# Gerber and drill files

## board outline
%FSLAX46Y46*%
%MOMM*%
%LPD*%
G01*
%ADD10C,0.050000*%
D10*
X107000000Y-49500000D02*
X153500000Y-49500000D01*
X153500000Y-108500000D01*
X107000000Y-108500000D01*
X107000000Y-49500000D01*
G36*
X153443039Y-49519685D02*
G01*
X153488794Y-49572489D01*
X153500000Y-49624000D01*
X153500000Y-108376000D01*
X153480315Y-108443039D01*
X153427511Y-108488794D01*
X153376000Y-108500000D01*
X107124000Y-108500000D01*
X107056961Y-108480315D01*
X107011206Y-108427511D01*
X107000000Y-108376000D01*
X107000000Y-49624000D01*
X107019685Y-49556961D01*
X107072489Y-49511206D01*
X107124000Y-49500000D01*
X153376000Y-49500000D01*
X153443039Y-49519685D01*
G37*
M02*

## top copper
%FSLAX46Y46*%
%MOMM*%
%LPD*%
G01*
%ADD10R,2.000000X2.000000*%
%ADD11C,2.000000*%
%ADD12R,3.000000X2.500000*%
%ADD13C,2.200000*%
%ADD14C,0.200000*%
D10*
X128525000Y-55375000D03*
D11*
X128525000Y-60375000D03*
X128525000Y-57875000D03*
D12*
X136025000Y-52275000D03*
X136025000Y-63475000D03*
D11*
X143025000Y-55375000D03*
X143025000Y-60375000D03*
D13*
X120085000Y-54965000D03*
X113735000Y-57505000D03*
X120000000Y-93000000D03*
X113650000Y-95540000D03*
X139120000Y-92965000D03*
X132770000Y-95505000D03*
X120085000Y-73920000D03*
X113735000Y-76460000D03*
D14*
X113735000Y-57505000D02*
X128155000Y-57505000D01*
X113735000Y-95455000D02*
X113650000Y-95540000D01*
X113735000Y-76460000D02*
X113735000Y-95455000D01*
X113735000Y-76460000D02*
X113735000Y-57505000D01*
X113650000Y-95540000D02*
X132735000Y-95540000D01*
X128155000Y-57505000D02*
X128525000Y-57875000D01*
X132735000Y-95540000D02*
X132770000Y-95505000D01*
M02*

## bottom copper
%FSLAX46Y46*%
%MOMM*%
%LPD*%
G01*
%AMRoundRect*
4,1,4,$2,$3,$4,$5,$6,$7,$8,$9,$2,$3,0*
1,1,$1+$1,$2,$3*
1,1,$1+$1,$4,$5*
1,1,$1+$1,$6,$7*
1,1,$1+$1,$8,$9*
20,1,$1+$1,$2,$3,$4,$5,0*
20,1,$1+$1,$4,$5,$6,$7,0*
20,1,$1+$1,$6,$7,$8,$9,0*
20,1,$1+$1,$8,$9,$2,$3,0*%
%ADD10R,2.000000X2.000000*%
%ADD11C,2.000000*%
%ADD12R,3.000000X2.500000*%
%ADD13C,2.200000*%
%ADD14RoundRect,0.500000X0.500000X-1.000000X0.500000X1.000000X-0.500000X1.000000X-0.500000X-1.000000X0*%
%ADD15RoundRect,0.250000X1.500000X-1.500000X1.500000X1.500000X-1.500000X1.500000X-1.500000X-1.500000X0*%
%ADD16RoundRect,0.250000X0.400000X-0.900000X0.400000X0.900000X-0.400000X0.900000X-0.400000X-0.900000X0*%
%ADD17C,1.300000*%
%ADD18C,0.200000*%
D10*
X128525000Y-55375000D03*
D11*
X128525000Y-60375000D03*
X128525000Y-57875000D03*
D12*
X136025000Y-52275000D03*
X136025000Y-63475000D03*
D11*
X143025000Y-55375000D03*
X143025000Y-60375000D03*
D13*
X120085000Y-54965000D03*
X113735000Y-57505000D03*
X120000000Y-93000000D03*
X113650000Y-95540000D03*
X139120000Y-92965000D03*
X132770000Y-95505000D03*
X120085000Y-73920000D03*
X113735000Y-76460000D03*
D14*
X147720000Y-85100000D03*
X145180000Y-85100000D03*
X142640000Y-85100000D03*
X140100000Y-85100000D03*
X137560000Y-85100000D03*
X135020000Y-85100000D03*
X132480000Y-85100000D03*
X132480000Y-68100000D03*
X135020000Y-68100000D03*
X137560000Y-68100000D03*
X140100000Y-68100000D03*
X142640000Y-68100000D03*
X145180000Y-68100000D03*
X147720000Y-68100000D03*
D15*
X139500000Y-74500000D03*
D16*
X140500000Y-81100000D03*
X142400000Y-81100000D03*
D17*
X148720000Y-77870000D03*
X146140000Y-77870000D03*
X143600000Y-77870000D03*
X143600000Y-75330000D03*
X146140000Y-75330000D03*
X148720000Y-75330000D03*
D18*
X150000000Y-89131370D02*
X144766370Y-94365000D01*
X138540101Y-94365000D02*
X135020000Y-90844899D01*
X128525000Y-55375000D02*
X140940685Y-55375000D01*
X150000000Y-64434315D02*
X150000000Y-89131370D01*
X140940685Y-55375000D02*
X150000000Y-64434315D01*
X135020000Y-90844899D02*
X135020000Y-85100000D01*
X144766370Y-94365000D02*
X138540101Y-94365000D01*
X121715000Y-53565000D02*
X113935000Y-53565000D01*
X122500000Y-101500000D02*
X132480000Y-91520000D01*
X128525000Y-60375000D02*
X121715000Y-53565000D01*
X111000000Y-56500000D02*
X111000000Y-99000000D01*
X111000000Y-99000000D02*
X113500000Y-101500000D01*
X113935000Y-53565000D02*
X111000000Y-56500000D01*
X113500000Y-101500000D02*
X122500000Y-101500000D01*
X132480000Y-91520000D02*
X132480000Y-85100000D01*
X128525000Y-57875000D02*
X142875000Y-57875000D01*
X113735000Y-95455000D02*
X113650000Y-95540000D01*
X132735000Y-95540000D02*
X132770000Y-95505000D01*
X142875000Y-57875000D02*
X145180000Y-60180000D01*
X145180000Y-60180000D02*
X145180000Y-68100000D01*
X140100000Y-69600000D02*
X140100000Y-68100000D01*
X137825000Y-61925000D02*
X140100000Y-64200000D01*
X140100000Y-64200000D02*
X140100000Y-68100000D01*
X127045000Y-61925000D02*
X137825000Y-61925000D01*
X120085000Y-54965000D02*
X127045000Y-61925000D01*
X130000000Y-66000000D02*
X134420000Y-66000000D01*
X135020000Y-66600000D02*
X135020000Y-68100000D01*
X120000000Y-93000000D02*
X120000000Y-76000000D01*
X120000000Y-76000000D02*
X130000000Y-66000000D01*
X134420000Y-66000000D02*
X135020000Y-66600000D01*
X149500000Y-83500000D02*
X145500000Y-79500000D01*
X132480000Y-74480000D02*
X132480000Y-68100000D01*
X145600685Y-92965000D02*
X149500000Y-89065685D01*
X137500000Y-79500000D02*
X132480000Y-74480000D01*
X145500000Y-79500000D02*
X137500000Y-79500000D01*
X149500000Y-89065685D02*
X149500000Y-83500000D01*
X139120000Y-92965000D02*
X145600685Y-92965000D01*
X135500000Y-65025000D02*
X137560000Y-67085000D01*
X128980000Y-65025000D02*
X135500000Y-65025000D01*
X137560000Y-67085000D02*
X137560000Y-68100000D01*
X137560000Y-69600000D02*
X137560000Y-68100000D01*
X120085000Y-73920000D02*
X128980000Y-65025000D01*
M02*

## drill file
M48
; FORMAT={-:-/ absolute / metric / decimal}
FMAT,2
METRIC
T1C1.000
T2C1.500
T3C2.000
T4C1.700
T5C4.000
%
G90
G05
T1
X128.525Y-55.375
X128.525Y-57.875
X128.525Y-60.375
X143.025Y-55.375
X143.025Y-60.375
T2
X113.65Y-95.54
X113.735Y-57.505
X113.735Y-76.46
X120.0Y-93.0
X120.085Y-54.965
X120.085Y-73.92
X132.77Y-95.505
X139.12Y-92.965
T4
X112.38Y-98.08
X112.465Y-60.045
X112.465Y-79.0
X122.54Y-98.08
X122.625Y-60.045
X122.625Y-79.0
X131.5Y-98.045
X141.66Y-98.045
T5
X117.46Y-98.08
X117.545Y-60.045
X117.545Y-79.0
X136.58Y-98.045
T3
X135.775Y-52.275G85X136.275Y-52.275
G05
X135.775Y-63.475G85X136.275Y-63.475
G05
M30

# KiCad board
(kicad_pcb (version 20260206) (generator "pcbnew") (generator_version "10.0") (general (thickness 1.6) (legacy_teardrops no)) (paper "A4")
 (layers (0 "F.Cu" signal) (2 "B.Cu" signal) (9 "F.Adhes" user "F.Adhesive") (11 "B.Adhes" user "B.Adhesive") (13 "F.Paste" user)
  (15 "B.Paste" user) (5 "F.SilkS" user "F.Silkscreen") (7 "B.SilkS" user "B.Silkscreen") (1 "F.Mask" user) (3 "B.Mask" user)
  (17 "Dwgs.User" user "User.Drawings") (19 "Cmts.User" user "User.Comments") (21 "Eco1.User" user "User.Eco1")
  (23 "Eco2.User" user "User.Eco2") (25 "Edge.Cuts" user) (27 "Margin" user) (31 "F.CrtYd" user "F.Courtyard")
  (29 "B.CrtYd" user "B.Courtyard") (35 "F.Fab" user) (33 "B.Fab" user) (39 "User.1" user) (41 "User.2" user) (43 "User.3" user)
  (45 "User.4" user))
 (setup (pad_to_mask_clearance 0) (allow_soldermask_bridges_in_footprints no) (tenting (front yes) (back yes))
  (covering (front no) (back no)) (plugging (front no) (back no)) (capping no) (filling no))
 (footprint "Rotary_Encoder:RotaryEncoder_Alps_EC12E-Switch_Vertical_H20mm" (layer "F.Cu") (at 128.525 55.375)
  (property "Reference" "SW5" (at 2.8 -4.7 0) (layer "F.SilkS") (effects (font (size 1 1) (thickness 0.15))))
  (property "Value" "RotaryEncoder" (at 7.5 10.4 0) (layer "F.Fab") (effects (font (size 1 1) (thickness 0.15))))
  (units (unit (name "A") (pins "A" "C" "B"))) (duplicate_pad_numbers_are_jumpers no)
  (pad "A" thru_hole rect (at 0 0) (size 2 2) (drill 1) (layers "*.Cu" "*.Mask") (remove_unused_layers no) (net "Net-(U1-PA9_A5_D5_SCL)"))
  (pad "B" thru_hole circle (at 0 5) (size 2 2) (drill 1) (layers "*.Cu" "*.Mask") (remove_unused_layers no) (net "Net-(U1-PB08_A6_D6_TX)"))
  (pad "C" thru_hole circle (at 0 2.5) (size 2 2) (drill 1) (layers "*.Cu" "*.Mask") (remove_unused_layers no) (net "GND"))
  (pad "MP" thru_hole rect (at 7.5 -3.1) (size 3 2.5) (drill oval 2.5 2) (layers "*.Cu" "*.Mask") (remove_unused_layers no))
  (pad "MP" thru_hole rect (at 7.5 8.1) (size 3 2.5) (drill oval 2.5 2) (layers "*.Cu" "*.Mask") (remove_unused_layers no))
  (pad "S1" thru_hole circle (at 14.5 0) (size 2 2) (drill 1) (layers "*.Cu" "*.Mask") (remove_unused_layers no))
  (pad "S2" thru_hole circle (at 14.5 5) (size 2 2) (drill 1) (layers "*.Cu" "*.Mask") (remove_unused_layers no)))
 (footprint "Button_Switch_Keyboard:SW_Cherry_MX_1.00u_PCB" (layer "F.Cu") (at 120.085 54.965)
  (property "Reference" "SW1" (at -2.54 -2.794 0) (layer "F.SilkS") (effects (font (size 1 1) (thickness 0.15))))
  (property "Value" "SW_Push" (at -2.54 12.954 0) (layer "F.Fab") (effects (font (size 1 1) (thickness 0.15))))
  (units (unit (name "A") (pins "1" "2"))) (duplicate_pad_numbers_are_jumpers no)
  (pad "" np_thru_hole circle (at -7.62 5.08) (size 1.7 1.7) (drill 1.7) (layers "*.Cu" "*.Mask"))
  (pad "" np_thru_hole circle (at -2.54 5.08) (size 4 4) (drill 4) (layers "*.Cu" "*.Mask"))
  (pad "" np_thru_hole circle (at 2.54 5.08) (size 1.7 1.7) (drill 1.7) (layers "*.Cu" "*.Mask"))
  (pad "1" thru_hole circle (at 0 0) (size 2.2 2.2) (drill 1.5) (layers "*.Cu" "*.Mask") (remove_unused_layers no)
   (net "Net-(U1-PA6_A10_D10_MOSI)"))
  (pad "2" thru_hole circle (at -6.35 2.54) (size 2.2 2.2) (drill 1.5) (layers "*.Cu" "*.Mask") (remove_unused_layers no) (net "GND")))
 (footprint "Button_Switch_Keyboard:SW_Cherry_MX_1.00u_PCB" (layer "F.Cu") (at 120 93)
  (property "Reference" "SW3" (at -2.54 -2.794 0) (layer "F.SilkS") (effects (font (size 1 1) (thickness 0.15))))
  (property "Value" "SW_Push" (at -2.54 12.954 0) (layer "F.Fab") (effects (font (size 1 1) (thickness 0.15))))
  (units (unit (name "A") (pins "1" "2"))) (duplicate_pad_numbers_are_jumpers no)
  (pad "" np_thru_hole circle (at -7.62 5.08) (size 1.7 1.7) (drill 1.7) (layers "*.Cu" "*.Mask"))
  (pad "" np_thru_hole circle (at -2.54 5.08) (size 4 4) (drill 4) (layers "*.Cu" "*.Mask"))
  (pad "" np_thru_hole circle (at 2.54 5.08) (size 1.7 1.7) (drill 1.7) (layers "*.Cu" "*.Mask"))
  (pad "1" thru_hole circle (at 0 0) (size 2.2 2.2) (drill 1.5) (layers "*.Cu" "*.Mask") (remove_unused_layers no)
   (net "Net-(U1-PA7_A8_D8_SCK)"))
  (pad "2" thru_hole circle (at -6.35 2.54) (size 2.2 2.2) (drill 1.5) (layers "*.Cu" "*.Mask") (remove_unused_layers no) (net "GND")))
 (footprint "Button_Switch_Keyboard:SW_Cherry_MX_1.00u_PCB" (layer "F.Cu") (at 139.12 92.965)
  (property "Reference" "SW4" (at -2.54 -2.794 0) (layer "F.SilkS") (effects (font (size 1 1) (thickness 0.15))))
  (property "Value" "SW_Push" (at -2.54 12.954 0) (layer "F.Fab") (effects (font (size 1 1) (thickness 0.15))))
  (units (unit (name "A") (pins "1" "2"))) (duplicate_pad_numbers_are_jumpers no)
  (pad "" np_thru_hole circle (at -7.62 5.08) (size 1.7 1.7) (drill 1.7) (layers "*.Cu" "*.Mask"))
  (pad "" np_thru_hole circle (at -2.54 5.08) (size 4 4) (drill 4) (layers "*.Cu" "*.Mask"))
  (pad "" np_thru_hole circle (at 2.54 5.08) (size 1.7 1.7) (drill 1.7) (layers "*.Cu" "*.Mask"))
  (pad "1" thru_hole circle (at 0 0) (size 2.2 2.2) (drill 1.5) (layers "*.Cu" "*.Mask") (remove_unused_layers no)
   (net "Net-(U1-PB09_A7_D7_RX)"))
  (pad "2" thru_hole circle (at -6.35 2.54) (size 2.2 2.2) (drill 1.5) (layers "*.Cu" "*.Mask") (remove_unused_layers no) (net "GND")))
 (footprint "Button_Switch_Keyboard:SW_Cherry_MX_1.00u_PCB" (layer "F.Cu") (at 120.085 73.92)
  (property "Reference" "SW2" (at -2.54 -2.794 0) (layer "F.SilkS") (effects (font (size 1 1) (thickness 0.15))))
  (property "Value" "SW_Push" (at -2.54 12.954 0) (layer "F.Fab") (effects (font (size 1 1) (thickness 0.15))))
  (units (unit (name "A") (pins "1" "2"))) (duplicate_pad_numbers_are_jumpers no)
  (pad "" np_thru_hole circle (at -7.62 5.08) (size 1.7 1.7) (drill 1.7) (layers "*.Cu" "*.Mask"))
  (pad "" np_thru_hole circle (at -2.54 5.08) (size 4 4) (drill 4) (layers "*.Cu" "*.Mask"))
  (pad "" np_thru_hole circle (at 2.54 5.08) (size 1.7 1.7) (drill 1.7) (layers "*.Cu" "*.Mask"))
  (pad "1" thru_hole circle (at 0 0) (size 2.2 2.2) (drill 1.5) (layers "*.Cu" "*.Mask") (remove_unused_layers no)
   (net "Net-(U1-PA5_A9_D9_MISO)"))
  (pad "2" thru_hole circle (at -6.35 2.54) (size 2.2 2.2) (drill 1.5) (layers "*.Cu" "*.Mask") (remove_unused_layers no) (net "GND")))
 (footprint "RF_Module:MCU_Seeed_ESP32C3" (layer "B.Cu") (at 140.1 76.6 90)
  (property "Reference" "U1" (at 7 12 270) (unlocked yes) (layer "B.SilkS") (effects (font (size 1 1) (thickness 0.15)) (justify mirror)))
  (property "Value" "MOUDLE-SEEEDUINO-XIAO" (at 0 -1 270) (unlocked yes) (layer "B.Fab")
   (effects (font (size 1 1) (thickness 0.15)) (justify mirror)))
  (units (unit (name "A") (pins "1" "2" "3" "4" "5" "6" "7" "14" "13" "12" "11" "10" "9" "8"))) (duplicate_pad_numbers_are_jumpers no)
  (pad "" smd roundrect (at 1.1 -1.6 90) (size 1.5 1.5) (layers "B.Paste") (roundrect_rratio 0.1666666667))
  (pad "" smd roundrect (at 1.1 0.4 90) (size 1.5 1.5) (layers "B.Paste") (roundrect_rratio 0.1666666667))
  (pad "" smd roundrect (at 3.1 -1.6 90) (size 1.5 1.5) (layers "B.Paste") (roundrect_rratio 0.1666666667))
  (pad "" smd roundrect (at 3.1 0.4 90) (size 1.5 1.5) (layers "B.Paste") (roundrect_rratio 0.1666666667))
  (pad "1" smd roundrect (at -8.5 7.62 90) (size 3 2) (layers "B.Cu" "B.Mask" "B.Paste") (roundrect_rratio 0.25)
   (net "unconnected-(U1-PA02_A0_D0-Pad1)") (thermal_bridge_angle 45))
  (pad "2" smd roundrect (at -8.5 5.08 90) (size 3 2) (layers "B.Cu" "B.Mask" "B.Paste") (roundrect_rratio 0.25)
   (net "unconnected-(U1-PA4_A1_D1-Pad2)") (thermal_bridge_angle 45))
  (pad "3" smd roundrect (at -8.5 2.54 90) (size 3 2) (layers "B.Cu" "B.Mask" "B.Paste") (roundrect_rratio 0.25)
   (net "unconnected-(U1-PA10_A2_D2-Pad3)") (thermal_bridge_angle 45))
  (pad "4" smd roundrect (at -8.5 0 90) (size 3 2) (layers "B.Cu" "B.Mask" "B.Paste") (roundrect_rratio 0.25)
   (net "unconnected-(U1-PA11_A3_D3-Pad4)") (thermal_bridge_angle 45))
  (pad "5" smd roundrect (at -8.5 -2.54 90) (size 3 2) (layers "B.Cu" "B.Mask" "B.Paste") (roundrect_rratio 0.25)
   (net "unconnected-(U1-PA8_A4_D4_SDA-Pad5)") (thermal_bridge_angle 45))
  (pad "6" smd roundrect (at -8.5 -5.08 90) (size 3 2) (layers "B.Cu" "B.Mask" "B.Paste") (roundrect_rratio 0.25)
   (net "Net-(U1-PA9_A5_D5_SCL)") (thermal_bridge_angle 45))
  (pad "7" smd roundrect (at -8.5 -7.62 90) (size 3 2) (layers "B.Cu" "B.Mask" "B.Paste") (roundrect_rratio 0.25)
   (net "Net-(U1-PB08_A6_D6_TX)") (thermal_bridge_angle 45))
  (pad "8" smd roundrect (at 8.5 -7.62 90) (size 3 2) (layers "B.Cu" "B.Mask" "B.Paste") (roundrect_rratio 0.25)
   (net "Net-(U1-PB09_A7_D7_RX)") (thermal_bridge_angle 45))
  (pad "9" smd roundrect (at 8.5 -5.08 90) (size 3 2) (layers "B.Cu" "B.Mask" "B.Paste") (roundrect_rratio 0.25)
   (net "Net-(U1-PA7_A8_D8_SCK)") (thermal_bridge_angle 45))
  (pad "10" smd roundrect (at 8.5 -2.54 90) (size 3 2) (layers "B.Cu" "B.Mask" "B.Paste") (roundrect_rratio 0.25)
   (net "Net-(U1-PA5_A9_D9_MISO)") (thermal_bridge_angle 45))
  (pad "11" smd roundrect (at 8.5 0 90) (size 3 2) (layers "B.Cu" "B.Mask" "B.Paste") (roundrect_rratio 0.25)
   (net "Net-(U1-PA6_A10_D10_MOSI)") (thermal_bridge_angle 45))
  (pad "12" smd roundrect (at 8.5 2.54 90) (size 3 2) (layers "B.Cu" "B.Mask" "B.Paste") (roundrect_rratio 0.25)
   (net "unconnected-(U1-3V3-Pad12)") (thermal_bridge_angle 45))
  (pad "13" smd roundrect (at 8.5 5.08 90) (size 3 2) (layers "B.Cu" "B.Mask" "B.Paste") (roundrect_rratio 0.25) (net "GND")
   (thermal_bridge_angle 45))
  (pad "14" smd roundrect (at 8.5 7.62 90) (size 3 2) (layers "B.Cu" "B.Mask" "B.Paste") (roundrect_rratio 0.25)
   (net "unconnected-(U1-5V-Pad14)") (thermal_bridge_angle 45))
  (pad "15" smd roundrect (at 2.1 -0.6 90) (size 3.5 3.5) (layers "B.Cu" "B.Mask") (roundrect_rratio 0.07142857143))
  (pad "16" smd roundrect (at -4.5 0.4 90) (size 2.3 1.3) (layers "B.Cu" "B.Mask" "B.Paste") (roundrect_rratio 0.1923076923))
  (pad "17" smd roundrect (at -4.5 2.3 90) (size 2.3 1.3) (layers "B.Cu" "B.Mask" "B.Paste") (roundrect_rratio 0.1923076923))
  (pad "18" smd circle (at -1.27 8.62 90) (size 1.3 1.3) (layers "B.Cu" "B.Mask" "B.Paste"))
  (pad "19" smd circle (at -1.27 6.04 90) (size 1.3 1.3) (layers "B.Cu" "B.Mask" "B.Paste"))
  (pad "20" smd circle (at -1.27 3.5 90) (size 1.3 1.3) (layers "B.Cu" "B.Mask" "B.Paste"))
  (pad "21" smd circle (at 1.27 3.5 90) (size 1.3 1.3) (layers "B.Cu" "B.Mask" "B.Paste"))
  (pad "22" smd circle (at 1.27 6.04 90) (size 1.3 1.3) (layers "B.Cu" "B.Mask" "B.Paste"))
  (pad "23" smd circle (at 1.27 8.62 90) (size 1.3 1.3) (layers "B.Cu" "B.Mask" "B.Paste")))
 (gr_rect (start 107 49.5) (end 153.5 108.5) (stroke (width 0.05) (type default)) (fill no) (layer "Edge.Cuts"))
 (segment (start 150 89.13137) (end 144.76637 94.365) (width 0.2) (layer "B.Cu") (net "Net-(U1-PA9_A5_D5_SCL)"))
 (segment (start 138.540101 94.365) (end 135.02 90.844899) (width 0.2) (layer "B.Cu") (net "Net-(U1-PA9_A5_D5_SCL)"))
 (segment (start 128.525 55.375) (end 140.940685 55.375) (width 0.2) (layer "B.Cu") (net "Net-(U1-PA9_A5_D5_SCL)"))
 (segment (start 150 64.434315) (end 150 89.13137) (width 0.2) (layer "B.Cu") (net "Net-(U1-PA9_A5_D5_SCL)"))
 (segment (start 140.940685 55.375) (end 150 64.434315) (width 0.2) (layer "B.Cu") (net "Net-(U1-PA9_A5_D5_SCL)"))
 (segment (start 135.02 90.844899) (end 135.02 85.1) (width 0.2) (layer "B.Cu") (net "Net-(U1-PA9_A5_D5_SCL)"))
 (segment (start 144.76637 94.365) (end 138.540101 94.365) (width 0.2) (layer "B.Cu") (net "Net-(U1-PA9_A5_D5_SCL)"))
 (segment (start 121.715 53.565) (end 113.935 53.565) (width 0.2) (layer "B.Cu") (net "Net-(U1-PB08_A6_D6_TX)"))
 (segment (start 122.5 101.5) (end 132.48 91.52) (width 0.2) (layer "B.Cu") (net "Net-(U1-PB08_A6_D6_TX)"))
 (segment (start 128.525 60.375) (end 121.715 53.565) (width 0.2) (layer "B.Cu") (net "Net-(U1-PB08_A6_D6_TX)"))
 (segment (start 111 56.5) (end 111 99) (width 0.2) (layer "B.Cu") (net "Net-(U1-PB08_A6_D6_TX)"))
 (segment (start 111 99) (end 113.5 101.5) (width 0.2) (layer "B.Cu") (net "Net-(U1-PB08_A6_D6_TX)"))
 (segment (start 113.935 53.565) (end 111 56.5) (width 0.2) (layer "B.Cu") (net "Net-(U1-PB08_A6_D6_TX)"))
 (segment (start 113.5 101.5) (end 122.5 101.5) (width 0.2) (layer "B.Cu") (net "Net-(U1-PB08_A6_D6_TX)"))
 (segment (start 132.48 91.52) (end 132.48 85.1) (width 0.2) (layer "B.Cu") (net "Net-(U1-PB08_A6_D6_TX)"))
 (segment (start 113.735 57.505) (end 128.155 57.505) (width 0.2) (layer "F.Cu") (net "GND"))
 (segment (start 113.735 95.455) (end 113.65 95.54) (width 0.2) (layer "F.Cu") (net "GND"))
 (segment (start 113.735 76.46) (end 113.735 95.455) (width 0.2) (layer "F.Cu") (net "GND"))
 (segment (start 113.735 76.46) (end 113.735 57.505) (width 0.2) (layer "F.Cu") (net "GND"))
 (segment (start 113.65 95.54) (end 132.735 95.54) (width 0.2) (layer "F.Cu") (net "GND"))
 (segment (start 128.155 57.505) (end 128.525 57.875) (width 0.2) (layer "F.Cu") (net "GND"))
 (segment (start 132.735 95.54) (end 132.77 95.505) (width 0.2) (layer "F.Cu") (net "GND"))
 (segment (start 128.525 57.875) (end 142.875 57.875) (width 0.2) (layer "B.Cu") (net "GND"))
 (segment (start 113.735 95.455) (end 113.65 95.54) (width 0.2) (layer "B.Cu") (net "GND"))
 (segment (start 132.735 95.54) (end 132.77 95.505) (width 0.2) (layer "B.Cu") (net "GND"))
 (segment (start 142.875 57.875) (end 145.18 60.18) (width 0.2) (layer "B.Cu") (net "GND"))
 (segment (start 145.18 60.18) (end 145.18 68.1) (width 0.2) (layer "B.Cu") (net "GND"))
 (segment (start 140.1 69.6) (end 140.1 68.1) (width 0.2) (layer "B.Cu") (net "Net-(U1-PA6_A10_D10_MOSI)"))
 (segment (start 137.825 61.925) (end 140.1 64.2) (width 0.2) (layer "B.Cu") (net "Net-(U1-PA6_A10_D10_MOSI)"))
 (segment (start 140.1 64.2) (end 140.1 68.1) (width 0.2) (layer "B.Cu") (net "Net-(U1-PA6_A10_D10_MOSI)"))
 (segment (start 127.045 61.925) (end 137.825 61.925) (width 0.2) (layer "B.Cu") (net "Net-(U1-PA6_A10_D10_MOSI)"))
 (segment (start 120.085 54.965) (end 127.045 61.925) (width 0.2) (layer "B.Cu") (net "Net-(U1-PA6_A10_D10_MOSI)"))
 (segment (start 130 66) (end 134.42 66) (width 0.2) (layer "B.Cu") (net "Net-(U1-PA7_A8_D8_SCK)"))
 (segment (start 135.02 66.6) (end 135.02 68.1) (width 0.2) (layer "B.Cu") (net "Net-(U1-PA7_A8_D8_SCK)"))
 (segment (start 120 93) (end 120 76) (width 0.2) (layer "B.Cu") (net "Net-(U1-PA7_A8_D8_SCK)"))
 (segment (start 120 76) (end 130 66) (width 0.2) (layer "B.Cu") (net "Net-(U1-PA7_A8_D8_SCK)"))
 (segment (start 134.42 66) (end 135.02 66.6) (width 0.2) (layer "B.Cu") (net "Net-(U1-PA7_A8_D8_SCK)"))
 (segment (start 149.5 83.5) (end 145.5 79.5) (width 0.2) (layer "B.Cu") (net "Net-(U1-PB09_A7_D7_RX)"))
 (segment (start 132.48 74.48) (end 132.48 68.1) (width 0.2) (layer "B.Cu") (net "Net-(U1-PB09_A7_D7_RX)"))
 (segment (start 145.600685 92.965) (end 149.5 89.065685) (width 0.2) (layer "B.Cu") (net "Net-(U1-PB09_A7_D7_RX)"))
 (segment (start 137.5 79.5) (end 132.48 74.48) (width 0.2) (layer "B.Cu") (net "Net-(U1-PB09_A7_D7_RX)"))
 (segment (start 145.5 79.5) (end 137.5 79.5) (width 0.2) (layer "B.Cu") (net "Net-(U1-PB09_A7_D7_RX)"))
 (segment (start 149.5 89.065685) (end 149.5 83.5) (width 0.2) (layer "B.Cu") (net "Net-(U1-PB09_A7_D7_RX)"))
 (segment (start 139.12 92.965) (end 145.600685 92.965) (width 0.2) (layer "B.Cu") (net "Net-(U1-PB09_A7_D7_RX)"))
 (segment (start 135.5 65.025) (end 137.56 67.085) (width 0.2) (layer "B.Cu") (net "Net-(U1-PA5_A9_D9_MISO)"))
 (segment (start 128.98 65.025) (end 135.5 65.025) (width 0.2) (layer "B.Cu") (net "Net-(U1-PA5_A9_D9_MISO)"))
 (segment (start 137.56 67.085) (end 137.56 68.1) (width 0.2) (layer "B.Cu") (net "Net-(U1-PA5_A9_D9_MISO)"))
 (segment (start 137.56 69.6) (end 137.56 68.1) (width 0.2) (layer "B.Cu") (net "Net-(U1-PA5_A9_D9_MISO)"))
 (segment (start 120.085 73.92) (end 128.98 65.025) (width 0.2) (layer "B.Cu") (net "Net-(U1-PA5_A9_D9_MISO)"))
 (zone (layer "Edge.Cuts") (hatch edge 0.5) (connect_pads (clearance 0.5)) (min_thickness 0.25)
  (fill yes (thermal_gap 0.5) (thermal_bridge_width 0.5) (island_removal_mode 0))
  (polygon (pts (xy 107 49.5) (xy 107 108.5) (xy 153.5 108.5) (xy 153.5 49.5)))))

